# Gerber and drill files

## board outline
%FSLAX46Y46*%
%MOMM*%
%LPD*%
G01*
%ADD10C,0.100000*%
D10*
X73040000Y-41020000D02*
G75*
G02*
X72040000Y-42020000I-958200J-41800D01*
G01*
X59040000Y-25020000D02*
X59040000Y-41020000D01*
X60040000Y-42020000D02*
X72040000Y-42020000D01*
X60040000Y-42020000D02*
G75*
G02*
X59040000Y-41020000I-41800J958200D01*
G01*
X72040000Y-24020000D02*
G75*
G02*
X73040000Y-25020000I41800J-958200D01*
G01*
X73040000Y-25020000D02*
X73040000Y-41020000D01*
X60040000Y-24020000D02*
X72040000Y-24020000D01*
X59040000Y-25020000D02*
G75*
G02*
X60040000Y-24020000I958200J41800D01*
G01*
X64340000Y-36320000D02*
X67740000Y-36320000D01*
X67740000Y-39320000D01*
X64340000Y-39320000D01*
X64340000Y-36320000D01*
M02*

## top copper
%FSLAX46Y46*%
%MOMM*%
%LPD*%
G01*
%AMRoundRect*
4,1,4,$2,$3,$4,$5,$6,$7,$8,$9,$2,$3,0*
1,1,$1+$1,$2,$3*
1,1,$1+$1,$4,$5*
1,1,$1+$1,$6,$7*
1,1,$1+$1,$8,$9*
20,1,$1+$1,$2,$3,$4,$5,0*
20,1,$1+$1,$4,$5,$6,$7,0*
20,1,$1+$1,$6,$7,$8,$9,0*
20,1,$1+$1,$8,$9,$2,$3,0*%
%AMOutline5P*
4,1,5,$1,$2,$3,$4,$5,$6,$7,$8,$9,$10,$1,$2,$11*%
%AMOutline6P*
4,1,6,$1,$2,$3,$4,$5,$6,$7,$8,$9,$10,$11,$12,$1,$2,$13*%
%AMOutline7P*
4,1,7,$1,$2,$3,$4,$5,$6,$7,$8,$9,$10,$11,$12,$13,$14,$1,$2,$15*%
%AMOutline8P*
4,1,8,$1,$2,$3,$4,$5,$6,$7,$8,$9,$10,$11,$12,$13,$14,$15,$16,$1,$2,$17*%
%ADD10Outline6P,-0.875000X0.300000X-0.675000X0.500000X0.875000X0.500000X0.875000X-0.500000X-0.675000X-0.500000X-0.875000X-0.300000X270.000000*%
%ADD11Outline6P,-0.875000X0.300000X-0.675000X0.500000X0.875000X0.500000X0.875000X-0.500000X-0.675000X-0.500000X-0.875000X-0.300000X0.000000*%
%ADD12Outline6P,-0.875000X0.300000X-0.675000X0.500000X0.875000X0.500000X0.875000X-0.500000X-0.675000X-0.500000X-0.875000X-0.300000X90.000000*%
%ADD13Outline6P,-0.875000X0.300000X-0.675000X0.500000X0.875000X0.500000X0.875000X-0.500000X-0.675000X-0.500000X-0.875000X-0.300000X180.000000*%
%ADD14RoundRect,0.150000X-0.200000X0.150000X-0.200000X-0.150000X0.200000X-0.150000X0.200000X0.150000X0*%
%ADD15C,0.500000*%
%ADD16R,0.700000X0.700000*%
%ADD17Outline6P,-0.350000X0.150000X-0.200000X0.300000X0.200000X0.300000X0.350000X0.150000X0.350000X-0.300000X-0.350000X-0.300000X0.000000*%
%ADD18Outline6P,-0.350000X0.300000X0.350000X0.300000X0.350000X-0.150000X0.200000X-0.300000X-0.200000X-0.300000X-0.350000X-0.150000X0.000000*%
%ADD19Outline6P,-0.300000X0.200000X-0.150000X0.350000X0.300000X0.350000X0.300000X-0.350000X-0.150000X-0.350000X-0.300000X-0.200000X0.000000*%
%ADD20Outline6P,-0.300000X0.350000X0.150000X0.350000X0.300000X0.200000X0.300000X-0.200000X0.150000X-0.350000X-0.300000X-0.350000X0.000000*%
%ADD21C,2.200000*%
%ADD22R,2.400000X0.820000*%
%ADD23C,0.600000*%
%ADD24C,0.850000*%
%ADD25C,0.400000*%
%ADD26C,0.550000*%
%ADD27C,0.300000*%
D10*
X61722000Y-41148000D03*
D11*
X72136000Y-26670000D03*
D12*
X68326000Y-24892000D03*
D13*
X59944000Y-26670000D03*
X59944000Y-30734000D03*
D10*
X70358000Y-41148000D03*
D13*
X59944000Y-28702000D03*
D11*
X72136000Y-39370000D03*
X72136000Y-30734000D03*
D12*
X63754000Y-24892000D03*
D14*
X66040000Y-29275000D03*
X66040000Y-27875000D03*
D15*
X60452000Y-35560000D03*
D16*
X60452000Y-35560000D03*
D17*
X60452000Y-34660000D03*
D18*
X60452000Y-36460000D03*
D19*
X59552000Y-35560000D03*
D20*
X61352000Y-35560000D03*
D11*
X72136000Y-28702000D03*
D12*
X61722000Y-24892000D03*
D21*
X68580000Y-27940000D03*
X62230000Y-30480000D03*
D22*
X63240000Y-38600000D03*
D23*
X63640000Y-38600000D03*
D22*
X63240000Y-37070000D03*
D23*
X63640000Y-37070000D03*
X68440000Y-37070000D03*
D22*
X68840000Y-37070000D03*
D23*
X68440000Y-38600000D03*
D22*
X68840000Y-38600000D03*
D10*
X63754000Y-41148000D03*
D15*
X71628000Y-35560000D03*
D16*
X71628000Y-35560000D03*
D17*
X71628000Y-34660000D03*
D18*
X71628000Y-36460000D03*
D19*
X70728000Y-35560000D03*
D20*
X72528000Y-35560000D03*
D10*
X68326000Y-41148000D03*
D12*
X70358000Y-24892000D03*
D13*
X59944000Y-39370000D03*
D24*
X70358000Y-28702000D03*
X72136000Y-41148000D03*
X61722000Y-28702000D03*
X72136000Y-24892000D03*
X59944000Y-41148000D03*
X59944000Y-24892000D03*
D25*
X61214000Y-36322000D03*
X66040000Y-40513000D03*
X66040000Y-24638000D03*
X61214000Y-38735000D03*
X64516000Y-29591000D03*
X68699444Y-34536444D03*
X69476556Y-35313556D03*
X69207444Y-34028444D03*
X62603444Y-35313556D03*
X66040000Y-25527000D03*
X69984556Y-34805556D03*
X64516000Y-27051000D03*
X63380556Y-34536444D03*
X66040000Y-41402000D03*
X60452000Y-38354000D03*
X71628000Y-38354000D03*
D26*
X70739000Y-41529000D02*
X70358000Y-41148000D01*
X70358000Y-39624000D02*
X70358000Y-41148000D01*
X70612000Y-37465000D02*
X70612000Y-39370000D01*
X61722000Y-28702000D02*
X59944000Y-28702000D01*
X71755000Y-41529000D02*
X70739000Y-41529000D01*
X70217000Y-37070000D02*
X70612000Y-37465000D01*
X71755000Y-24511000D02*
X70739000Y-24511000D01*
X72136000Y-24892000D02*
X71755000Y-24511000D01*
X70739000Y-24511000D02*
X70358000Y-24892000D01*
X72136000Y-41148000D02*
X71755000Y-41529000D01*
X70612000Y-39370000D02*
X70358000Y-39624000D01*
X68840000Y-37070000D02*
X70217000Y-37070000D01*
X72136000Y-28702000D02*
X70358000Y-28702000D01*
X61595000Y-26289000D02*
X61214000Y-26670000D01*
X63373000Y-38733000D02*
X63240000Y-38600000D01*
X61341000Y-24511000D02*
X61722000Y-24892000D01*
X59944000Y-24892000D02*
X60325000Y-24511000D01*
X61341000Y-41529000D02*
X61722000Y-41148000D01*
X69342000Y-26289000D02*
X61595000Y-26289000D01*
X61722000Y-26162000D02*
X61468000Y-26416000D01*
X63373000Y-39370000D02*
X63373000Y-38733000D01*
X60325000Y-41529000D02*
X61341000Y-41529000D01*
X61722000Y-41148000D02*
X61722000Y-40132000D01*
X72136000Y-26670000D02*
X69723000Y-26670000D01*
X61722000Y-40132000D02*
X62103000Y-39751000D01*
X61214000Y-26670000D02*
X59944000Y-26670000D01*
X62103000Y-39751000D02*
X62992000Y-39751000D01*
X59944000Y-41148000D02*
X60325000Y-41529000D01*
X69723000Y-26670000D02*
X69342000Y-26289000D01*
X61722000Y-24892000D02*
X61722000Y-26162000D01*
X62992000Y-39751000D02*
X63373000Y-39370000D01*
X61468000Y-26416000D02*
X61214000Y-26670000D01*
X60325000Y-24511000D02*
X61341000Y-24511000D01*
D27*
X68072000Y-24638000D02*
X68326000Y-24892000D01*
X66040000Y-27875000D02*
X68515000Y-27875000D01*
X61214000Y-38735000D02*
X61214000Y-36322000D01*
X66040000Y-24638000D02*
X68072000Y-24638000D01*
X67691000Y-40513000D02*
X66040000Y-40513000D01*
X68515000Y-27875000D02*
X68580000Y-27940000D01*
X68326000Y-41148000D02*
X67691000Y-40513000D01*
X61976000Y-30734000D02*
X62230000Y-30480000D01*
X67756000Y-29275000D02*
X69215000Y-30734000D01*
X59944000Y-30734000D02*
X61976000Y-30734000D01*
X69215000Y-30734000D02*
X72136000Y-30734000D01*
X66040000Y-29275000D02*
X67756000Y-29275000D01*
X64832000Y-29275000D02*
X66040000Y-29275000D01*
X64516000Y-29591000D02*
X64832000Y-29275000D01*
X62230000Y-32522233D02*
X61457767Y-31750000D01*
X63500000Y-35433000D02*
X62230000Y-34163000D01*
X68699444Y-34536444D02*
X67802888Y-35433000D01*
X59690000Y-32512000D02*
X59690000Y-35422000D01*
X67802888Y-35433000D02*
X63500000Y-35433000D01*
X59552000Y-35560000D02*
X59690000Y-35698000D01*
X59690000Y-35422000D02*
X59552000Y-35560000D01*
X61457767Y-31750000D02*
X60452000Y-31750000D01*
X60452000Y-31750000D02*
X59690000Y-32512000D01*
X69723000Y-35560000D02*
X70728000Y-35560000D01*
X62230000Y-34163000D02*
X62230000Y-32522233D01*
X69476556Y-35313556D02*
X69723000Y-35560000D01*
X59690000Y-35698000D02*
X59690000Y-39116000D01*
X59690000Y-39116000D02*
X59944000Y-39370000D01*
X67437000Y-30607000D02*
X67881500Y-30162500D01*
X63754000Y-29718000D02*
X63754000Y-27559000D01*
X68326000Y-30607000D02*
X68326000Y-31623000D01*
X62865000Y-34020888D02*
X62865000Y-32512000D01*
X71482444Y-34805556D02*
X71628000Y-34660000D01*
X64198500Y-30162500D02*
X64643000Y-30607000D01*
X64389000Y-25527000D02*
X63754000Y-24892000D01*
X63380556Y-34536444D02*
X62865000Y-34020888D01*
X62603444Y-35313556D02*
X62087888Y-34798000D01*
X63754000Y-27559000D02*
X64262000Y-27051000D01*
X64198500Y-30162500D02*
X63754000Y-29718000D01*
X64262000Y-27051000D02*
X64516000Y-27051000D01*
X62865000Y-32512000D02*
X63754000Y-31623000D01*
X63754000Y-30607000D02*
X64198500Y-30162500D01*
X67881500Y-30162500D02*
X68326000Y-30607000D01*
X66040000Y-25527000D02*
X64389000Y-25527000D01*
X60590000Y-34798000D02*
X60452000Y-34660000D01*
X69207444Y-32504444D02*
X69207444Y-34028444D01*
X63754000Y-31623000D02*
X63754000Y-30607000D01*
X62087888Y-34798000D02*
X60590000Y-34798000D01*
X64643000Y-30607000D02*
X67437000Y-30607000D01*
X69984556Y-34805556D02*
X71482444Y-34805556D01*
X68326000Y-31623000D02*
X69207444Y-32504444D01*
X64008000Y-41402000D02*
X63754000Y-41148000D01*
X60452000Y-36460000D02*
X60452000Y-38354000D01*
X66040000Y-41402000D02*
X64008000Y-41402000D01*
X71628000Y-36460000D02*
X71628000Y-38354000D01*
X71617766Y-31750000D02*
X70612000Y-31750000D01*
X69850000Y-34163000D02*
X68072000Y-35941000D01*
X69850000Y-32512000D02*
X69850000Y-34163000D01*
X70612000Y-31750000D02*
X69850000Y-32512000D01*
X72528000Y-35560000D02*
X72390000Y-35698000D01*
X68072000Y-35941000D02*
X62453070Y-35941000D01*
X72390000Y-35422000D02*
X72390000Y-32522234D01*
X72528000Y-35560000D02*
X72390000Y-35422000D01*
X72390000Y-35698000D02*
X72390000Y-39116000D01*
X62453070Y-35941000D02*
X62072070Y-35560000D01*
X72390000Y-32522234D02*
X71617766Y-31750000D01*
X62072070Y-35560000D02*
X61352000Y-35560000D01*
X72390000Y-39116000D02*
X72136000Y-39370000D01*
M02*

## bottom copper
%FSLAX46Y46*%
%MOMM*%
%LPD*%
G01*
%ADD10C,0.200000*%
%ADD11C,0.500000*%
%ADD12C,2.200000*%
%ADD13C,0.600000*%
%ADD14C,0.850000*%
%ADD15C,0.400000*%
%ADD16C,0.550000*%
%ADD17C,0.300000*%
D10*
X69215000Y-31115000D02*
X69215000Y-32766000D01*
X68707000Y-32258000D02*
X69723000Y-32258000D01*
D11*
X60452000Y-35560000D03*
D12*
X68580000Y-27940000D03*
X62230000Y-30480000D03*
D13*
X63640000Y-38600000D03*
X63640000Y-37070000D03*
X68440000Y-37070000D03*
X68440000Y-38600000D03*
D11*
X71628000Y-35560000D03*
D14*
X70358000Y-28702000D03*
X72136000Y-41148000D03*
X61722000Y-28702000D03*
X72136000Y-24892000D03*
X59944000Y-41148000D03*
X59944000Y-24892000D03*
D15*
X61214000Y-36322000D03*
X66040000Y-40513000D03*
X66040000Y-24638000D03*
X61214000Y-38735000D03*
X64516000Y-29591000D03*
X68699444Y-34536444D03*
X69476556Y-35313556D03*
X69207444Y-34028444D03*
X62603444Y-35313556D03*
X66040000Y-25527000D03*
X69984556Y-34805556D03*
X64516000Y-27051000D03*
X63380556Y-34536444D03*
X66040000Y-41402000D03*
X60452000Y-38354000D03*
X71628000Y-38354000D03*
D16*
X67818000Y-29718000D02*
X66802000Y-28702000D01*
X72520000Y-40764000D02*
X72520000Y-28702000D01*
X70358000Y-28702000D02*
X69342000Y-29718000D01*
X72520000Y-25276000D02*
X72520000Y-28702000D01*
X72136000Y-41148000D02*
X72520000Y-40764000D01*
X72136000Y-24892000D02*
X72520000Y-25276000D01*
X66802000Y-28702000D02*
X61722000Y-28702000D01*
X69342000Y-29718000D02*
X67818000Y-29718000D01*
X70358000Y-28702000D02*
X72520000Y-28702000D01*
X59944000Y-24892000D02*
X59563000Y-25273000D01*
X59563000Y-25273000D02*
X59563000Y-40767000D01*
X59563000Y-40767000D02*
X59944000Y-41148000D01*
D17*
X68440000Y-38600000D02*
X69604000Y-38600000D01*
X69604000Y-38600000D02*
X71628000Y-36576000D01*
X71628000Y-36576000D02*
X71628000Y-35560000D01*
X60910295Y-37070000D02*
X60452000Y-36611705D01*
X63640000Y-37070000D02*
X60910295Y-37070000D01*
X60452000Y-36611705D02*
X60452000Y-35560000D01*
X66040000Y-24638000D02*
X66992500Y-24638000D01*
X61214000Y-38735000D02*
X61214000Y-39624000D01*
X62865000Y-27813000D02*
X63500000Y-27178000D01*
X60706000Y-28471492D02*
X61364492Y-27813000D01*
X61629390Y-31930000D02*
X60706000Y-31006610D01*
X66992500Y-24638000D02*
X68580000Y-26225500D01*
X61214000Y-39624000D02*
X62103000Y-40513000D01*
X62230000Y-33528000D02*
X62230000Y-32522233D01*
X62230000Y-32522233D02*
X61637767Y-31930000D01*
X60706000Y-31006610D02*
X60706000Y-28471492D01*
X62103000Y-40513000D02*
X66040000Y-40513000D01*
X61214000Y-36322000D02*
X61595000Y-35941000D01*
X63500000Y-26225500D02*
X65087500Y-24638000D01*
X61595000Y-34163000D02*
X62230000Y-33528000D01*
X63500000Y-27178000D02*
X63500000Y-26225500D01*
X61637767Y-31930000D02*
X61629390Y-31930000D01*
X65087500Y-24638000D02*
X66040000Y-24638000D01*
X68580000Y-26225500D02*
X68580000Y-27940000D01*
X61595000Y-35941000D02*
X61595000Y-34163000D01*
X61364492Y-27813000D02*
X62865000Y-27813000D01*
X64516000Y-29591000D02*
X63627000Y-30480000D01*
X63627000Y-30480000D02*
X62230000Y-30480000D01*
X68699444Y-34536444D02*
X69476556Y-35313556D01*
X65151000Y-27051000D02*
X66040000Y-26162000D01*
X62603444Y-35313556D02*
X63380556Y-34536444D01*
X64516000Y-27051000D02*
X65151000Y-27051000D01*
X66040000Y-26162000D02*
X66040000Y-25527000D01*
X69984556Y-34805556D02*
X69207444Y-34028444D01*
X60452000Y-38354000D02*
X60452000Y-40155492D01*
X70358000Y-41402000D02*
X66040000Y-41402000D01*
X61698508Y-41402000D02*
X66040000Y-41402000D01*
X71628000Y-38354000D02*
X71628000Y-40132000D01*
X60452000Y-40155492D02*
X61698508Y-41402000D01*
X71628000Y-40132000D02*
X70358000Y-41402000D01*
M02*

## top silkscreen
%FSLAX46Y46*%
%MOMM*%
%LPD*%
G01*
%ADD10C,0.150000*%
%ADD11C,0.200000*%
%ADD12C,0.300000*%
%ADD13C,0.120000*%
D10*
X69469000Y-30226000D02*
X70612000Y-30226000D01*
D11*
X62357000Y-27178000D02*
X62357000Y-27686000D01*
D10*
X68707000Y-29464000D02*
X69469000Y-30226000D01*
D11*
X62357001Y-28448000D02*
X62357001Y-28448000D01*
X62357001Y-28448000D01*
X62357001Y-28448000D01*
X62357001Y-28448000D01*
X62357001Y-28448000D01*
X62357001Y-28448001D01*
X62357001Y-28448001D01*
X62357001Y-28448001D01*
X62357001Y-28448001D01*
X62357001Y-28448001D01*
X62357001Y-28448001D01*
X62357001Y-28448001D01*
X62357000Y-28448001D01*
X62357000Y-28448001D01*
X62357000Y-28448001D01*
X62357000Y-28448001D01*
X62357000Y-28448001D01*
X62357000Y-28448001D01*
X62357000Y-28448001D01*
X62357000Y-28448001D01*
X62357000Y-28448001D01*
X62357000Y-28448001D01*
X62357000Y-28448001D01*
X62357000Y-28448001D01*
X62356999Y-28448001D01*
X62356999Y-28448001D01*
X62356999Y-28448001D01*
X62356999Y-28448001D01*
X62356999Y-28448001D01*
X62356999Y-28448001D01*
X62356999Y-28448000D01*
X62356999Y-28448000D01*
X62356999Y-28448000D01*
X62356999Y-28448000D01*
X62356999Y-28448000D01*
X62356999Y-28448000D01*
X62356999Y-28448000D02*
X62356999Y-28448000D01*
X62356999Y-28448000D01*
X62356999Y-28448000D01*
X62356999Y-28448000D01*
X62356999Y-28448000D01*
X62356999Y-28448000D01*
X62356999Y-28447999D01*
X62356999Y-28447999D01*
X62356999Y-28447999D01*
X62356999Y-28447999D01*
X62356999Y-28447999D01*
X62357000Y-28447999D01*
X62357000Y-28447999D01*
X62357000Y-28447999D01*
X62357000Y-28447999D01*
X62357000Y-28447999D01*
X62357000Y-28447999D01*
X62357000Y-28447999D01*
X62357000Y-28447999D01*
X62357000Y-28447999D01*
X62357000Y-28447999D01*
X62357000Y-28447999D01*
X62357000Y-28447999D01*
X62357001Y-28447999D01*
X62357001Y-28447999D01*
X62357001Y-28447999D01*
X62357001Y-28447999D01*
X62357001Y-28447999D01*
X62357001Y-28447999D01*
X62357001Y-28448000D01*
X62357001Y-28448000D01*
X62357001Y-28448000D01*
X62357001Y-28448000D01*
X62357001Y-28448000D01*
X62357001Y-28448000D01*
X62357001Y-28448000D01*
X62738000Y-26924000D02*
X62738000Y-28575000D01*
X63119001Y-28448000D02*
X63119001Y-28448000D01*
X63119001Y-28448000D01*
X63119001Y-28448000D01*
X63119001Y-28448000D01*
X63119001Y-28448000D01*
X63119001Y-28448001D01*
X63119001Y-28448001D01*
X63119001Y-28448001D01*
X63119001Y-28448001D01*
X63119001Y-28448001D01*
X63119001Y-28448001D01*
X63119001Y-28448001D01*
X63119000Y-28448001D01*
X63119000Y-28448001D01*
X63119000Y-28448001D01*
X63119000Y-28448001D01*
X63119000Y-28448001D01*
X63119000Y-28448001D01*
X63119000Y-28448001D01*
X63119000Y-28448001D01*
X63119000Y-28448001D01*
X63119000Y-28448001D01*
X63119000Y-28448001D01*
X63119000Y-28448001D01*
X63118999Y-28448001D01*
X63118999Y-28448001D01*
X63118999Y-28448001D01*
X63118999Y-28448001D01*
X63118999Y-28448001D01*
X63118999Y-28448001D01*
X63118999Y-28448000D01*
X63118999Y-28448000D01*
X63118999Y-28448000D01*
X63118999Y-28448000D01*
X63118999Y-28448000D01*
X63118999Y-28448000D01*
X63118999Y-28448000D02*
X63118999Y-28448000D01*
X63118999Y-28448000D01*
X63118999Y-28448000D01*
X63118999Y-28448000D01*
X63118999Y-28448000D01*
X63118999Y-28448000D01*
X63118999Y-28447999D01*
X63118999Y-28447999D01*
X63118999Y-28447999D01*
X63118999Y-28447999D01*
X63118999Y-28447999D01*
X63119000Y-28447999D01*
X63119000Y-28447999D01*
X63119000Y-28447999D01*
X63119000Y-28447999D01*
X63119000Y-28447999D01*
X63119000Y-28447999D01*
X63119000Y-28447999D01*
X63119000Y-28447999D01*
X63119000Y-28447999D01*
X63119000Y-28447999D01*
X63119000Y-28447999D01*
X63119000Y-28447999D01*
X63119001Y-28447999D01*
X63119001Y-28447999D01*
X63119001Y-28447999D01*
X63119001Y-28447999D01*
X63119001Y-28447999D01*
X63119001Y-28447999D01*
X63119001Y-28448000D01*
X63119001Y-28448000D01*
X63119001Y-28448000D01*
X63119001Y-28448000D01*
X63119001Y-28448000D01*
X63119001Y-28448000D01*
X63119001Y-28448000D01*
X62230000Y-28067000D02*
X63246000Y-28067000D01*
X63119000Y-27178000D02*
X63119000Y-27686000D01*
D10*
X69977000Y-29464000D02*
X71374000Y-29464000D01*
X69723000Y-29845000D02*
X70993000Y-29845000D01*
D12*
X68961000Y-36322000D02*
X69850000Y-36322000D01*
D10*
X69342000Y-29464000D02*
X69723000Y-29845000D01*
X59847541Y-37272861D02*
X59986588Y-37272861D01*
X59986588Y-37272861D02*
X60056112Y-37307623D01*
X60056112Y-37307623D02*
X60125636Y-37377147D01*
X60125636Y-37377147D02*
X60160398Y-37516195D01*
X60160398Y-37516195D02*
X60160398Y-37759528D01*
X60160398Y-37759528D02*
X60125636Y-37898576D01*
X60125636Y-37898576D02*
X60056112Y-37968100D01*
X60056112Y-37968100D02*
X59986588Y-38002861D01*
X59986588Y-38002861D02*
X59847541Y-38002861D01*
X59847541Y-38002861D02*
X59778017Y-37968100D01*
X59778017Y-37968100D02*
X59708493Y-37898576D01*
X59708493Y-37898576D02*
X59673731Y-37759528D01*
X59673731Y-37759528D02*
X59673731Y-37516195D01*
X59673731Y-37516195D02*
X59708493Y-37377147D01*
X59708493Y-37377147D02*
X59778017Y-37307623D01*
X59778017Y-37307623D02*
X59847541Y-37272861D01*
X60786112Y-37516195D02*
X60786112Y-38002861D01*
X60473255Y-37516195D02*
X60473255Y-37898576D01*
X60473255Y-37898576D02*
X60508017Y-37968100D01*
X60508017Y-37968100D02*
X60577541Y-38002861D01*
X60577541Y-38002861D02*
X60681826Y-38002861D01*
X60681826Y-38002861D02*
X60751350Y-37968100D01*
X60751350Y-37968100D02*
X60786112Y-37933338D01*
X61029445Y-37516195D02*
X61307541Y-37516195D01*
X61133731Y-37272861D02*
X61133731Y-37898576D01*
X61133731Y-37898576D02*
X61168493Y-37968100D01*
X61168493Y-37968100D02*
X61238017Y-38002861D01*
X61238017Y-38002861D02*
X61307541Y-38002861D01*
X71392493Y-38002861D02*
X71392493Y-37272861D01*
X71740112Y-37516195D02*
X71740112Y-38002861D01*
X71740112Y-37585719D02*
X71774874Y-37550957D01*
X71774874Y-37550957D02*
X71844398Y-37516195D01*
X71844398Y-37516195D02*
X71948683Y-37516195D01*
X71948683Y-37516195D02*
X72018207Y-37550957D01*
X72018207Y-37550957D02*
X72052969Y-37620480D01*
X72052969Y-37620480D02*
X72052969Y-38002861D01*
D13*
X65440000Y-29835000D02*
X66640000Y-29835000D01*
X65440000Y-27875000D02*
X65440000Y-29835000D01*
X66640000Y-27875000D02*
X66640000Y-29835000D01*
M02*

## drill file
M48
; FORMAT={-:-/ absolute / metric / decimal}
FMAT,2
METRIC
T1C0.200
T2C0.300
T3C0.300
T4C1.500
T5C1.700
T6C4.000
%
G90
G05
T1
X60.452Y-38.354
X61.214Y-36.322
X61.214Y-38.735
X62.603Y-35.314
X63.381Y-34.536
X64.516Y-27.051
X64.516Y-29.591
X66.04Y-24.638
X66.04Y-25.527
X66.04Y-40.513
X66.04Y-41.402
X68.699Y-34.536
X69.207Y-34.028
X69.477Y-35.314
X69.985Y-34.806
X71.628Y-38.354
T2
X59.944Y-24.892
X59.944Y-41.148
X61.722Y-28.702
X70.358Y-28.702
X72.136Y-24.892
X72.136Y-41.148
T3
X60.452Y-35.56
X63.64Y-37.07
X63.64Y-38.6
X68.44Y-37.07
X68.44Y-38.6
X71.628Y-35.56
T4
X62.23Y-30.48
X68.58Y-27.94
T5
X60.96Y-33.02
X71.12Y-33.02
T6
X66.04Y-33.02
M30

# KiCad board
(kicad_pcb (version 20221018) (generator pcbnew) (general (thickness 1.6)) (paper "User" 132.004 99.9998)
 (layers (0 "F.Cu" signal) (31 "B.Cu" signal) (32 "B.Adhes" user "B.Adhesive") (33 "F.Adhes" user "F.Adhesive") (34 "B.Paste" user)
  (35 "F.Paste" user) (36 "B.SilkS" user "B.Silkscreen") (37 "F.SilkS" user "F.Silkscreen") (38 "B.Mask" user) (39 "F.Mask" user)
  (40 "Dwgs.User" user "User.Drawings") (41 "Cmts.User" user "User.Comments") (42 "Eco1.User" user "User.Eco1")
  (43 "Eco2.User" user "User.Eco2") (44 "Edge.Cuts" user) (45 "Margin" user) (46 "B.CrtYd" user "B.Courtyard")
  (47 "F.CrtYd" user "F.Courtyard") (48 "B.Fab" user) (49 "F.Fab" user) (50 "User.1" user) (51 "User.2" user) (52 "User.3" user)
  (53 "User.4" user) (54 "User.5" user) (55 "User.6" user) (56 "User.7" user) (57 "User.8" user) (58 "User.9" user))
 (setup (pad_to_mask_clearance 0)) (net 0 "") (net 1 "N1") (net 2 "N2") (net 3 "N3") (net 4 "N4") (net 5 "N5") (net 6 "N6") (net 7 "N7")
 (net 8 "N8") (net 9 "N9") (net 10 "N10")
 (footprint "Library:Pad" (layer "F.Cu") (at 61.722 41.148 -90)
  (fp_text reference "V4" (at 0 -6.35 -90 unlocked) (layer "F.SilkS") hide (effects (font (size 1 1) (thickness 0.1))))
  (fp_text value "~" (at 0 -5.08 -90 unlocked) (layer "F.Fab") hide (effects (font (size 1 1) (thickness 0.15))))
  (pad "1" smd roundrect (at 0 0 270) (size 1.75 1) (layers "F.Cu" "F.Paste" "F.Mask") (roundrect_rratio 0) (chamfer_ratio 0.2)
   (chamfer top_left bottom_left) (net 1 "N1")))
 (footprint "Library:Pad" (layer "F.Cu") (at 72.136 26.67)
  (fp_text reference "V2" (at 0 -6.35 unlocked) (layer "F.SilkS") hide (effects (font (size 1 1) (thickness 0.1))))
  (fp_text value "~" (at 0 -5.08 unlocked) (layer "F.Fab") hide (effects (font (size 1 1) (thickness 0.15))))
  (pad "1" smd roundrect (at 0 0) (size 1.75 1) (layers "F.Cu" "F.Paste" "F.Mask") (roundrect_rratio 0) (chamfer_ratio 0.2)
   (chamfer top_left bottom_left) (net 1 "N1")))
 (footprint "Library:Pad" (layer "F.Cu") (at 68.326 24.892 90)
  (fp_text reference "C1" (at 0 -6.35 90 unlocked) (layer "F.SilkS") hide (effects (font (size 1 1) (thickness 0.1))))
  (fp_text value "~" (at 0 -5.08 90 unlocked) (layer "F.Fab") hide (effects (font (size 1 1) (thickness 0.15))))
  (pad "1" smd roundrect (at 0 0 90) (size 1.75 1) (layers "F.Cu" "F.Paste" "F.Mask") (roundrect_rratio 0) (chamfer_ratio 0.2)
   (chamfer top_left bottom_left) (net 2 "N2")))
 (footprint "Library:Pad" (layer "F.Cu") (at 59.944 26.67 180)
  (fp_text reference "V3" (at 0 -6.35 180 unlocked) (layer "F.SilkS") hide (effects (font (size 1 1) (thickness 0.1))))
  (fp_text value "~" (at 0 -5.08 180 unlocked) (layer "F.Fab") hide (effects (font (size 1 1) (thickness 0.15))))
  (pad "1" smd roundrect (at 0 0 180) (size 1.75 1) (layers "F.Cu" "F.Paste" "F.Mask") (roundrect_rratio 0) (chamfer_ratio 0.2)
   (chamfer top_left bottom_left) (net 1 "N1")))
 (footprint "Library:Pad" (layer "F.Cu") (at 59.944 30.734 180)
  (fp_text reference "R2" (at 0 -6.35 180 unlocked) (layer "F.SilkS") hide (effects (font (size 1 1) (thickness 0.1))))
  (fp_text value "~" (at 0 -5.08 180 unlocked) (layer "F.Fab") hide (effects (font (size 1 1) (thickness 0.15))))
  (pad "1" smd roundrect (at 0 0 180) (size 1.75 1) (layers "F.Cu" "F.Paste" "F.Mask") (roundrect_rratio 0) (chamfer_ratio 0.2)
   (chamfer top_left bottom_left) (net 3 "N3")))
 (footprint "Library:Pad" (layer "F.Cu") (at 70.358 41.148 -90)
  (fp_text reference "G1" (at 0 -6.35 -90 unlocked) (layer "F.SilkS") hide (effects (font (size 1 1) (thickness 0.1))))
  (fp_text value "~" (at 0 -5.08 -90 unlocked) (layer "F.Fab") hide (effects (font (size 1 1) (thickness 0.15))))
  (pad "1" smd roundrect (at 0 0 270) (size 1.75 1) (layers "F.Cu" "F.Paste" "F.Mask") (roundrect_rratio 0) (chamfer_ratio 0.2)
   (chamfer top_left bottom_left) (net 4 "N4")))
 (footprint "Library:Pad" (layer "F.Cu") (at 59.944 28.702 180)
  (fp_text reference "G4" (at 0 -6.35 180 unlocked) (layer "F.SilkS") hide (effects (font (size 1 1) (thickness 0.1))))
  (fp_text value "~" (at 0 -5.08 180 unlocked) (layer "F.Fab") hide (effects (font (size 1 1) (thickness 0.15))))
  (pad "1" smd roundrect (at 0 0 180) (size 1.75 1) (layers "F.Cu" "F.Paste" "F.Mask") (roundrect_rratio 0) (chamfer_ratio 0.2)
   (chamfer top_left bottom_left) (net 4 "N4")))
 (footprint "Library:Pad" (layer "F.Cu") (at 72.136 39.37)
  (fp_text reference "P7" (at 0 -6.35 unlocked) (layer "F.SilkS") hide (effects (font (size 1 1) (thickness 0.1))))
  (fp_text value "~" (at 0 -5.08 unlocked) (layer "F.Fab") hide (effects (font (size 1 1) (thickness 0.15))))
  (pad "1" smd roundrect (at 0 0) (size 1.75 1) (layers "F.Cu" "F.Paste" "F.Mask") (roundrect_rratio 0) (chamfer_ratio 0.2)
   (chamfer top_left bottom_left) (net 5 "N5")))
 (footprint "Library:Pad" (layer "F.Cu") (at 72.136 30.734)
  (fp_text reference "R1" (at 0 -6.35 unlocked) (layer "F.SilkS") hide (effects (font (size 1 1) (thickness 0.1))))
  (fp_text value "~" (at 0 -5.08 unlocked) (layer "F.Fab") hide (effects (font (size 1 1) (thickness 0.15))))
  (pad "1" smd roundrect (at 0 0) (size 1.75 1) (layers "F.Cu" "F.Paste" "F.Mask") (roundrect_rratio 0) (chamfer_ratio 0.2)
   (chamfer top_left bottom_left) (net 3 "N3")))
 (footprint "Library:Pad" (layer "F.Cu") (at 63.754 24.892 90)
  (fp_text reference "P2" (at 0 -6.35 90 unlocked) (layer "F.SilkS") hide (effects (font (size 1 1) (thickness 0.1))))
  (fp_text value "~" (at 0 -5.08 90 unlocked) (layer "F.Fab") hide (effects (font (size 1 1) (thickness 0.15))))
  (pad "1" smd roundrect (at 0 0 90) (size 1.75 1) (layers "F.Cu" "F.Paste" "F.Mask") (roundrect_rratio 0) (chamfer_ratio 0.2)
   (chamfer top_left bottom_left) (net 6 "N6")))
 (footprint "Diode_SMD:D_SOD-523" (layer "F.Cu") (at 66.04 28.575 90)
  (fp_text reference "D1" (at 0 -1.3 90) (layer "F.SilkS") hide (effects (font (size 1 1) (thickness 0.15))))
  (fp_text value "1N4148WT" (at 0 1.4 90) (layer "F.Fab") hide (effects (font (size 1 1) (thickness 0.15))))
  (fp_line (start -1.26 -0.6) (end -1.26 0.6) (stroke (width 0.12) (type solid)) (layer "F.SilkS"))
  (fp_line (start 0.7 -0.6) (end -1.26 -0.6) (stroke (width 0.12) (type solid)) (layer "F.SilkS"))
  (fp_line (start 0.7 0.6) (end -1.26 0.6) (stroke (width 0.12) (type solid)) (layer "F.SilkS"))
  (pad "1" smd roundrect (at -0.7 0 270) (size 0.6 0.7) (layers "F.Cu" "F.Paste" "F.Mask") (roundrect_rratio 0.25) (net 3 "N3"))
  (pad "2" smd roundrect (at 0.7 0 270) (size 0.6 0.7) (layers "F.Cu" "F.Paste" "F.Mask") (roundrect_rratio 0.25) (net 2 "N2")))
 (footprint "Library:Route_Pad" (layer "F.Cu") (at 60.452 35.56)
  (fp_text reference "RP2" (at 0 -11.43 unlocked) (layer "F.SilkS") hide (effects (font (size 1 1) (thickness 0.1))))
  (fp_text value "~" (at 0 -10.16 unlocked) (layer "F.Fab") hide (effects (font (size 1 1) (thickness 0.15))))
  (pad "1" thru_hole circle (at 0 0) (size 0.5 0.5) (drill 0.3) (layers "*.Cu" "*.Mask") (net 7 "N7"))
  (pad "1" smd rect (at 0 0) (size 0.7 0.7) (layers "F.Cu" "F.Paste" "F.Mask") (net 7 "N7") (thermal_bridge_angle 45))
  (pad "2" smd roundrect (at 0 -0.9) (size 0.7 0.6) (layers "F.Cu" "F.Paste" "F.Mask") (roundrect_rratio 0) (chamfer_ratio 0.25)
   (chamfer top_left top_right) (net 6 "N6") (thermal_bridge_angle 45))
  (pad "3" smd roundrect (at 0 0.9) (size 0.7 0.6) (layers "F.Cu" "F.Paste" "F.Mask") (roundrect_rratio 0) (chamfer_ratio 0.25)
   (chamfer bottom_left bottom_right) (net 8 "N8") (thermal_bridge_angle 45))
  (pad "4" smd roundrect (at -0.9 0) (size 0.6 0.7) (layers "F.Cu" "F.Paste" "F.Mask") (roundrect_rratio 0) (chamfer_ratio 0.25)
   (chamfer top_left bottom_left) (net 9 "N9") (thermal_bridge_angle 45))
  (pad "5" smd roundrect (at 0.9 0) (size 0.6 0.7) (layers "F.Cu" "F.Paste" "F.Mask") (roundrect_rratio 0) (chamfer_ratio 0.25)
   (chamfer top_right bottom_right) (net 5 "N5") (thermal_bridge_angle 45)))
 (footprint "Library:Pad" (layer "F.Cu") (at 72.136 28.702)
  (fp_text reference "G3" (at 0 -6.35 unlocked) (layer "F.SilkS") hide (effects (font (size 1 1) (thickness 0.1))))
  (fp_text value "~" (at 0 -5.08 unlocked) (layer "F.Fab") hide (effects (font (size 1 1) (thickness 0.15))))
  (pad "1" smd roundrect (at 0 0) (size 1.75 1) (layers "F.Cu" "F.Paste" "F.Mask") (roundrect_rratio 0) (chamfer_ratio 0.2)
   (chamfer top_left bottom_left) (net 4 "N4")))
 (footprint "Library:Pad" (layer "F.Cu") (at 61.722 24.892 90)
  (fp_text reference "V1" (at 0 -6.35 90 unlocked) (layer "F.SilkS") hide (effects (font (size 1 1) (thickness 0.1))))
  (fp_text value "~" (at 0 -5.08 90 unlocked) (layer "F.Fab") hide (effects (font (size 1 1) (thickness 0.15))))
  (pad "1" smd roundrect (at 0 0 90) (size 1.75 1) (layers "F.Cu" "F.Paste" "F.Mask") (roundrect_rratio 0) (chamfer_ratio 0.2)
   (chamfer top_left bottom_left) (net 1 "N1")))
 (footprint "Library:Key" (layer "F.Cu") (at 66.04 33.02)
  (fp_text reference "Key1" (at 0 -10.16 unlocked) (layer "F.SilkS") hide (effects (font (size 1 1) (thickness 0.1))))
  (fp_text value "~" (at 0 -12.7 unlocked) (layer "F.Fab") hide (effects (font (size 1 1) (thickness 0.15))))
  (fp_rect (start -1.7 3.3) (end 1.7 6.3) (stroke (width 0.1) (type default)) (fill none) (layer "Edge.Cuts"))
  (pad "" np_thru_hole circle (at -5.08 0) (size 1.7 1.7) (drill 1.7) (layers "F&B.Cu" "*.Mask"))
  (pad "" np_thru_hole circle (at 0 0) (size 4 4) (drill 4) (layers "F&B.Cu" "*.Mask"))
  (pad "" np_thru_hole circle (at 5.08 0) (size 1.7 1.7) (drill 1.7) (layers "F&B.Cu" "*.Mask"))
  (pad "1" thru_hole circle (at 2.54 -5.08) (size 2.2 2.2) (drill 1.5) (layers "*.Cu" "*.Mask") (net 2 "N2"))
  (pad "2" thru_hole circle (at -3.81 -2.54) (size 2.2 2.2) (drill 1.5) (layers "*.Cu" "*.Mask") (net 3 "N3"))
  (pad "3" smd rect (at -2.8 5.58) (size 2.4 0.82) (layers "F.Cu" "F.Paste" "F.Mask") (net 1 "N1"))
  (pad "3" thru_hole circle (at -2.4 5.58) (size 0.6 0.6) (drill 0.3) (layers "*.Cu" "*.Mask") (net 1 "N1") (thermal_bridge_angle 90))
  (pad "4" smd rect (at -2.8 4.05) (size 2.4 0.82) (layers "F.Cu" "F.Paste" "F.Mask") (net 7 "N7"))
  (pad "4" thru_hole circle (at -2.4 4.05) (size 0.6 0.6) (drill 0.3) (layers "*.Cu" "*.Mask") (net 7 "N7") (thermal_bridge_angle 90))
  (pad "5" thru_hole circle (at 2.4 4.05) (size 0.6 0.6) (drill 0.3) (layers "*.Cu" "*.Mask") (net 4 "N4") (thermal_bridge_angle 90))
  (pad "5" smd rect (at 2.8 4.05) (size 2.4 0.82) (layers "F.Cu" "F.Paste" "F.Mask") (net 4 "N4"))
  (pad "6" thru_hole circle (at 2.4 5.58) (size 0.6 0.6) (drill 0.3) (layers "*.Cu" "*.Mask") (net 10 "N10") (thermal_bridge_angle 90))
  (pad "6" smd rect (at 2.8 5.58) (size 2.4 0.82) (layers "F.Cu" "F.Paste" "F.Mask") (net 10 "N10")))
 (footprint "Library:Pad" (layer "F.Cu") (at 63.754 41.148 -90)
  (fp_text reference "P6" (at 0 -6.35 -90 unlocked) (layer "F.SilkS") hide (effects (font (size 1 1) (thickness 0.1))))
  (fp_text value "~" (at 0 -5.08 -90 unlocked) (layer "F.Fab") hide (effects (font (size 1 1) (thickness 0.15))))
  (pad "1" smd roundrect (at 0 0 270) (size 1.75 1) (layers "F.Cu" "F.Paste" "F.Mask") (roundrect_rratio 0) (chamfer_ratio 0.2)
   (chamfer top_left bottom_left) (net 8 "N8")))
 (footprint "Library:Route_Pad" (layer "F.Cu") (at 71.628 35.56)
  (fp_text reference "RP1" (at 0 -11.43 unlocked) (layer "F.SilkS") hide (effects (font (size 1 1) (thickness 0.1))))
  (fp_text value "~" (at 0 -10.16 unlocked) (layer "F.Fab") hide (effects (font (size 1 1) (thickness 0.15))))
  (pad "1" thru_hole circle (at 0 0) (size 0.5 0.5) (drill 0.3) (layers "*.Cu" "*.Mask") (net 10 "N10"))
  (pad "1" smd rect (at 0 0) (size 0.7 0.7) (layers "F.Cu" "F.Paste" "F.Mask") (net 10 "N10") (thermal_bridge_angle 45))
  (pad "2" smd roundrect (at 0 -0.9) (size 0.7 0.6) (layers "F.Cu" "F.Paste" "F.Mask") (roundrect_rratio 0) (chamfer_ratio 0.25)
   (chamfer top_left top_right) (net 6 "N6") (thermal_bridge_angle 45))
  (pad "3" smd roundrect (at 0 0.9) (size 0.7 0.6) (layers "F.Cu" "F.Paste" "F.Mask") (roundrect_rratio 0) (chamfer_ratio 0.25)
   (chamfer bottom_left bottom_right) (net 8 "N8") (thermal_bridge_angle 45))
  (pad "4" smd roundrect (at -0.9 0) (size 0.6 0.7) (layers "F.Cu" "F.Paste" "F.Mask") (roundrect_rratio 0) (chamfer_ratio 0.25)
   (chamfer top_left bottom_left) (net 9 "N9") (thermal_bridge_angle 45))
  (pad "5" smd roundrect (at 0.9 0) (size 0.6 0.7) (layers "F.Cu" "F.Paste" "F.Mask") (roundrect_rratio 0) (chamfer_ratio 0.25)
   (chamfer top_right bottom_right) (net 5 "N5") (thermal_bridge_angle 45)))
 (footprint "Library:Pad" (layer "F.Cu") (at 68.326 41.148 -90)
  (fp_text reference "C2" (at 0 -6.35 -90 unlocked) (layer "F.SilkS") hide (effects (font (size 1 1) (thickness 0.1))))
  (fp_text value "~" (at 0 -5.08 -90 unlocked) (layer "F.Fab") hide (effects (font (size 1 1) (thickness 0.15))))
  (pad "1" smd roundrect (at 0 0 270) (size 1.75 1) (layers "F.Cu" "F.Paste" "F.Mask") (roundrect_rratio 0) (chamfer_ratio 0.2)
   (chamfer top_left bottom_left) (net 2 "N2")))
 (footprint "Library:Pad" (layer "F.Cu") (at 70.358 24.892 90)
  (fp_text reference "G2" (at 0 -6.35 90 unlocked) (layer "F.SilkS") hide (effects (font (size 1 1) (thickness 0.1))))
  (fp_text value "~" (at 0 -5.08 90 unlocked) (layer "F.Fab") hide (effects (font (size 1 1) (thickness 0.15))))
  (pad "1" smd roundrect (at 0 0 90) (size 1.75 1) (layers "F.Cu" "F.Paste" "F.Mask") (roundrect_rratio 0) (chamfer_ratio 0.2)
   (chamfer top_left bottom_left) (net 4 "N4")))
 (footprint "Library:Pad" (layer "F.Cu") (at 59.944 39.37 180)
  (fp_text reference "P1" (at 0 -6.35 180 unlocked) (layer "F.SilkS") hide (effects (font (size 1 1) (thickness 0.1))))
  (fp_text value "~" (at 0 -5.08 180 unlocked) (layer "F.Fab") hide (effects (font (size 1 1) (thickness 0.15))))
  (pad "1" smd roundrect (at 0 0 180) (size 1.75 1) (layers "F.Cu" "F.Paste" "F.Mask") (roundrect_rratio 0) (chamfer_ratio 0.2)
   (chamfer top_left bottom_left) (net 9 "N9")))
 (gr_line (start 69.215 31.115) (end 69.215 32.766) (stroke (width 0.2) (type default)) (layer "B.Cu"))
 (gr_line (start 68.707 32.258) (end 69.723 32.258) (stroke (width 0.2) (type default)) (layer "B.Cu"))
 (gr_line (start 69.469 30.226) (end 70.612 30.226) (stroke (width 0.15) (type default)) (layer "F.SilkS"))
 (gr_line (start 62.357 27.178) (end 62.357 27.686) (stroke (width 0.2) (type default)) (layer "F.SilkS"))
 (gr_line (start 68.707 29.464) (end 69.469 30.226) (stroke (width 0.15) (type default)) (layer "F.SilkS"))
 (gr_circle (center 62.357 28.448) (end 62.357001 28.448) (stroke (width 0.2) (type default)) (fill none) (layer "F.SilkS"))
 (gr_line (start 62.738 26.924) (end 62.738 28.575) (stroke (width 0.2) (type default)) (layer "F.SilkS"))
 (gr_circle (center 63.119 28.448) (end 63.119001 28.448) (stroke (width 0.2) (type default)) (fill none) (layer "F.SilkS"))
 (gr_line (start 62.23 28.067) (end 63.246 28.067) (stroke (width 0.2) (type default)) (layer "F.SilkS"))
 (gr_line (start 63.119 27.178) (end 63.119 27.686) (stroke (width 0.2) (type default)) (layer "F.SilkS"))
 (gr_line (start 69.977 29.464) (end 71.374 29.464) (stroke (width 0.15) (type default)) (layer "F.SilkS"))
 (gr_line (start 69.723 29.845) (end 70.993 29.845) (stroke (width 0.15) (type default)) (layer "F.SilkS"))
 (gr_line (start 68.961 36.322) (end 69.85 36.322) (stroke (width 0.3) (type default)) (layer "F.SilkS"))
 (gr_line (start 69.342 29.464) (end 69.723 29.845) (stroke (width 0.15) (type default)) (layer "F.SilkS"))
 (gr_arc (start 73.04 41.02) (mid 72.759994 41.739993) (end 72.04 42.02) (stroke (width 0.1) (type default)) (layer "Edge.Cuts"))
 (gr_line (start 59.04 25.02) (end 59.04 41.02) (stroke (width 0.1) (type default)) (layer "Edge.Cuts"))
 (gr_line (start 60.04 42.02) (end 72.04 42.02) (stroke (width 0.1) (type default)) (layer "Edge.Cuts"))
 (gr_arc (start 60.04 42.02) (mid 59.320007 41.739994) (end 59.04 41.02) (stroke (width 0.1) (type default)) (layer "Edge.Cuts"))
 (gr_arc (start 72.04 24.02) (mid 72.759993 24.300006) (end 73.04 25.02) (stroke (width 0.1) (type default)) (layer "Edge.Cuts"))
 (gr_line (start 73.04 25.02) (end 73.04 41.02) (stroke (width 0.1) (type default)) (layer "Edge.Cuts"))
 (gr_line (start 60.04 24.02) (end 72.04 24.02) (stroke (width 0.1) (type default)) (layer "Edge.Cuts"))
 (gr_arc (start 59.04 25.02) (mid 59.320006 24.300007) (end 60.04 24.02) (stroke (width 0.1) (type default)) (layer "Edge.Cuts"))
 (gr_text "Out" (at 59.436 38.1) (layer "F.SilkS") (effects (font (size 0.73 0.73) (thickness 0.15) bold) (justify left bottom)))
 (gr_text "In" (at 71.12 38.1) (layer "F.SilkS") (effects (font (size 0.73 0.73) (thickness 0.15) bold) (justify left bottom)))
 (segment (start 70.739 41.529) (end 70.358 41.148) (width 0.55) (layer "F.Cu") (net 4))
 (segment (start 70.358 39.624) (end 70.358 41.148) (width 0.55) (layer "F.Cu") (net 4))
 (segment (start 70.612 37.465) (end 70.612 39.37) (width 0.55) (layer "F.Cu") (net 4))
 (segment (start 61.722 28.702) (end 59.944 28.702) (width 0.55) (layer "F.Cu") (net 4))
 (segment (start 71.755 41.529) (end 70.739 41.529) (width 0.55) (layer "F.Cu") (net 4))
 (segment (start 70.217 37.07) (end 70.612 37.465) (width 0.55) (layer "F.Cu") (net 4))
 (segment (start 71.755 24.511) (end 70.739 24.511) (width 0.55) (layer "F.Cu") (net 4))
 (segment (start 72.136 24.892) (end 71.755 24.511) (width 0.55) (layer "F.Cu") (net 4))
 (segment (start 70.739 24.511) (end 70.358 24.892) (width 0.55) (layer "F.Cu") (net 4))
 (segment (start 72.136 41.148) (end 71.755 41.529) (width 0.55) (layer "F.Cu") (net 4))
 (segment (start 70.612 39.37) (end 70.358 39.624) (width 0.55) (layer "F.Cu") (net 4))
 (segment (start 68.84 37.07) (end 70.217 37.07) (width 0.55) (layer "F.Cu") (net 4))
 (segment (start 72.136 28.702) (end 70.358 28.702) (width 0.55) (layer "F.Cu") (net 4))
 (via (at 70.358 28.702) (size 0.85) (drill 0.3) (layers "F.Cu" "B.Cu") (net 4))
 (via (at 72.136 41.148) (size 0.85) (drill 0.3) (layers "F.Cu" "B.Cu") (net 4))
 (via (at 61.722 28.702) (size 0.85) (drill 0.3) (layers "F.Cu" "B.Cu") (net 4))
 (via (at 72.136 24.892) (size 0.85) (drill 0.3) (layers "F.Cu" "B.Cu") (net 4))
 (segment (start 67.818 29.718) (end 66.802 28.702) (width 0.55) (layer "B.Cu") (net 4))
 (segment (start 72.52 40.764) (end 72.52 28.702) (width 0.55) (layer "B.Cu") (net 4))
 (segment (start 70.358 28.702) (end 69.342 29.718) (width 0.55) (layer "B.Cu") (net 4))
 (segment (start 72.52 25.276) (end 72.52 28.702) (width 0.55) (layer "B.Cu") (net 4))
 (segment (start 72.136 41.148) (end 72.52 40.764) (width 0.55) (layer "B.Cu") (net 4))
 (segment (start 72.136 24.892) (end 72.52 25.276) (width 0.55) (layer "B.Cu") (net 4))
 (segment (start 66.802 28.702) (end 61.722 28.702) (width 0.55) (layer "B.Cu") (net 4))
 (segment (start 69.342 29.718) (end 67.818 29.718) (width 0.55) (layer "B.Cu") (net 4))
 (segment (start 70.358 28.702) (end 72.52 28.702) (width 0.55) (layer "B.Cu") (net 4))
 (segment (start 61.595 26.289) (end 61.214 26.67) (width 0.55) (layer "F.Cu") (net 1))
 (segment (start 63.373 38.733) (end 63.24 38.6) (width 0.55) (layer "F.Cu") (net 1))
 (segment (start 61.341 24.511) (end 61.722 24.892) (width 0.55) (layer "F.Cu") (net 1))
 (segment (start 59.944 24.892) (end 60.325 24.511) (width 0.55) (layer "F.Cu") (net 1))
 (segment (start 61.341 41.529) (end 61.722 41.148) (width 0.55) (layer "F.Cu") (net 1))
 (segment (start 69.342 26.289) (end 61.595 26.289) (width 0.55) (layer "F.Cu") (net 1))
 (segment (start 61.722 26.162) (end 61.468 26.416) (width 0.55) (layer "F.Cu") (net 1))
 (segment (start 63.373 39.37) (end 63.373 38.733) (width 0.55) (layer "F.Cu") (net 1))
 (segment (start 60.325 41.529) (end 61.341 41.529) (width 0.55) (layer "F.Cu") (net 1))
 (segment (start 61.722 41.148) (end 61.722 40.132) (width 0.55) (layer "F.Cu") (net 1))
 (segment (start 72.136 26.67) (end 69.723 26.67) (width 0.55) (layer "F.Cu") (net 1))
 (segment (start 61.722 40.132) (end 62.103 39.751) (width 0.55) (layer "F.Cu") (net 1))
 (segment (start 61.214 26.67) (end 59.944 26.67) (width 0.55) (layer "F.Cu") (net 1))
 (segment (start 62.103 39.751) (end 62.992 39.751) (width 0.55) (layer "F.Cu") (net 1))
 (segment (start 59.944 41.148) (end 60.325 41.529) (width 0.55) (layer "F.Cu") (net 1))
 (segment (start 69.723 26.67) (end 69.342 26.289) (width 0.55) (layer "F.Cu") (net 1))
 (segment (start 61.722 24.892) (end 61.722 26.162) (width 0.55) (layer "F.Cu") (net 1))
 (segment (start 62.992 39.751) (end 63.373 39.37) (width 0.55) (layer "F.Cu") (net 1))
 (segment (start 61.468 26.416) (end 61.214 26.67) (width 0.55) (layer "F.Cu") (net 1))
 (segment (start 60.325 24.511) (end 61.341 24.511) (width 0.55) (layer "F.Cu") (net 1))
 (via (at 59.944 41.148) (size 0.85) (drill 0.3) (layers "F.Cu" "B.Cu") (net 1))
 (via (at 59.944 24.892) (size 0.85) (drill 0.3) (layers "F.Cu" "B.Cu") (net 1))
 (segment (start 59.944 24.892) (end 59.563 25.273) (width 0.55) (layer "B.Cu") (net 1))
 (segment (start 59.563 25.273) (end 59.563 40.767) (width 0.55) (layer "B.Cu") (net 1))
 (segment (start 59.563 40.767) (end 59.944 41.148) (width 0.55) (layer "B.Cu") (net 1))
 (segment (start 68.44 38.6) (end 69.604 38.6) (width 0.3) (layer "B.Cu") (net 10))
 (segment (start 69.604 38.6) (end 71.628 36.576) (width 0.3) (layer "B.Cu") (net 10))
 (segment (start 71.628 36.576) (end 71.628 35.56) (width 0.3) (layer "B.Cu") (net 10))
 (segment (start 60.910295 37.07) (end 60.452 36.611705) (width 0.3) (layer "B.Cu") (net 7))
 (segment (start 63.64 37.07) (end 60.910295 37.07) (width 0.3) (layer "B.Cu") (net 7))
 (segment (start 60.452 36.611705) (end 60.452 35.56) (width 0.3) (layer "B.Cu") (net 7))
 (segment (start 68.072 24.638) (end 68.326 24.892) (width 0.3) (layer "F.Cu") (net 2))
 (segment (start 66.04 27.875) (end 68.515 27.875) (width 0.3) (layer "F.Cu") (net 2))
 (segment (start 61.214 38.735) (end 61.214 36.322) (width 0.3) (layer "F.Cu") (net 2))
 (segment (start 66.04 24.638) (end 68.072 24.638) (width 0.3) (layer "F.Cu") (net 2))
 (segment (start 67.691 40.513) (end 66.04 40.513) (width 0.3) (layer "F.Cu") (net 2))
 (segment (start 68.515 27.875) (end 68.58 27.94) (width 0.3) (layer "F.Cu") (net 2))
 (segment (start 68.326 41.148) (end 67.691 40.513) (width 0.3) (layer "F.Cu") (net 2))
 (via (at 61.214 36.322) (size 0.4) (drill 0.2) (layers "F.Cu" "B.Cu") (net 2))
 (via (at 66.04 40.513) (size 0.4) (drill 0.2) (layers "F.Cu" "B.Cu") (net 2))
 (via (at 66.04 24.638) (size 0.4) (drill 0.2) (layers "F.Cu" "B.Cu") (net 2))
 (via (at 61.214 38.735) (size 0.4) (drill 0.2) (layers "F.Cu" "B.Cu") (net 2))
 (segment (start 66.04 24.638) (end 66.9925 24.638) (width 0.3) (layer "B.Cu") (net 2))
 (segment (start 61.214 38.735) (end 61.214 39.624) (width 0.3) (layer "B.Cu") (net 2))
 (segment (start 62.865 27.813) (end 63.5 27.178) (width 0.3) (layer "B.Cu") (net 2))
 (segment (start 60.706 28.471492) (end 61.364492 27.813) (width 0.3) (layer "B.Cu") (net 2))
 (segment (start 61.62939 31.93) (end 60.706 31.00661) (width 0.3) (layer "B.Cu") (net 2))
 (segment (start 66.9925 24.638) (end 68.58 26.2255) (width 0.3) (layer "B.Cu") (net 2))
 (segment (start 61.214 39.624) (end 62.103 40.513) (width 0.3) (layer "B.Cu") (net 2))
 (segment (start 62.23 33.528) (end 62.23 32.522233) (width 0.3) (layer "B.Cu") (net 2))
 (segment (start 62.23 32.522233) (end 61.637767 31.93) (width 0.3) (layer "B.Cu") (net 2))
 (segment (start 60.706 31.00661) (end 60.706 28.471492) (width 0.3) (layer "B.Cu") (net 2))
 (segment (start 62.103 40.513) (end 66.04 40.513) (width 0.3) (layer "B.Cu") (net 2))
 (segment (start 61.214 36.322) (end 61.595 35.941) (width 0.3) (layer "B.Cu") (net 2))
 (segment (start 63.5 26.2255) (end 65.0875 24.638) (width 0.3) (layer "B.Cu") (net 2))
 (segment (start 61.595 34.163) (end 62.23 33.528) (width 0.3) (layer "B.Cu") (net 2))
 (segment (start 63.5 27.178) (end 63.5 26.2255) (width 0.3) (layer "B.Cu") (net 2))
 (segment (start 61.637767 31.93) (end 61.62939 31.93) (width 0.3) (layer "B.Cu") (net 2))
 (segment (start 65.0875 24.638) (end 66.04 24.638) (width 0.3) (layer "B.Cu") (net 2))
 (segment (start 68.58 26.2255) (end 68.58 27.94) (width 0.3) (layer "B.Cu") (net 2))
 (segment (start 61.595 35.941) (end 61.595 34.163) (width 0.3) (layer "B.Cu") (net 2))
 (segment (start 61.364492 27.813) (end 62.865 27.813) (width 0.3) (layer "B.Cu") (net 2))
 (segment (start 61.976 30.734) (end 62.23 30.48) (width 0.3) (layer "F.Cu") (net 3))
 (segment (start 67.756 29.275) (end 69.215 30.734) (width 0.3) (layer "F.Cu") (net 3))
 (segment (start 59.944 30.734) (end 61.976 30.734) (width 0.3) (layer "F.Cu") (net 3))
 (segment (start 69.215 30.734) (end 72.136 30.734) (width 0.3) (layer "F.Cu") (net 3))
 (segment (start 66.04 29.275) (end 67.756 29.275) (width 0.3) (layer "F.Cu") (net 3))
 (segment (start 64.832 29.275) (end 66.04 29.275) (width 0.3) (layer "F.Cu") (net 3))
 (segment (start 64.516 29.591) (end 64.832 29.275) (width 0.3) (layer "F.Cu") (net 3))
 (via (at 64.516 29.591) (size 0.4) (drill 0.2) (layers "F.Cu" "B.Cu") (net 3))
 (segment (start 64.516 29.591) (end 63.627 30.48) (width 0.3) (layer "B.Cu") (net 3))
 (segment (start 63.627 30.48) (end 62.23 30.48) (width 0.3) (layer "B.Cu") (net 3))
 (segment (start 62.23 32.522233) (end 61.457767 31.75) (width 0.3) (layer "F.Cu") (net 9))
 (segment (start 63.5 35.433) (end 62.23 34.163) (width 0.3) (layer "F.Cu") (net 9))
 (segment (start 68.699444 34.536444) (end 67.802888 35.433) (width 0.3) (layer "F.Cu") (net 9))
 (segment (start 59.69 32.512) (end 59.69 35.422) (width 0.3) (layer "F.Cu") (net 9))
 (segment (start 67.802888 35.433) (end 63.5 35.433) (width 0.3) (layer "F.Cu") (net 9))
 (segment (start 59.552 35.56) (end 59.69 35.698) (width 0.3) (layer "F.Cu") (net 9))
 (segment (start 59.69 35.422) (end 59.552 35.56) (width 0.3) (layer "F.Cu") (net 9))
 (segment (start 61.457767 31.75) (end 60.452 31.75) (width 0.3) (layer "F.Cu") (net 9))
 (segment (start 60.452 31.75) (end 59.69 32.512) (width 0.3) (layer "F.Cu") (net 9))
 (segment (start 69.723 35.56) (end 70.728 35.56) (width 0.3) (layer "F.Cu") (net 9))
 (segment (start 62.23 34.163) (end 62.23 32.522233) (width 0.3) (layer "F.Cu") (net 9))
 (segment (start 69.476556 35.313556) (end 69.723 35.56) (width 0.3) (layer "F.Cu") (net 9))
 (segment (start 59.69 35.698) (end 59.69 39.116) (width 0.3) (layer "F.Cu") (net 9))
 (segment (start 59.69 39.116) (end 59.944 39.37) (width 0.3) (layer "F.Cu") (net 9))
 (via (at 68.699444 34.536444) (size 0.4) (drill 0.2) (layers "F.Cu" "B.Cu") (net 9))
 (via (at 69.476556 35.313556) (size 0.4) (drill 0.2) (layers "F.Cu" "B.Cu") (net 9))
 (segment (start 68.699444 34.536444) (end 69.476556 35.313556) (width 0.3) (layer "B.Cu") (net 9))
 (segment (start 67.437 30.607) (end 67.8815 30.1625) (width 0.3) (layer "F.Cu") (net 6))
 (segment (start 63.754 29.718) (end 63.754 27.559) (width 0.3) (layer "F.Cu") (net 6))
 (segment (start 68.326 30.607) (end 68.326 31.623) (width 0.3) (layer "F.Cu") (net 6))
 (segment (start 62.865 34.020888) (end 62.865 32.512) (width 0.3) (layer "F.Cu") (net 6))
 (segment (start 71.482444 34.805556) (end 71.628 34.66) (width 0.3) (layer "F.Cu") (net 6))
 (segment (start 64.1985 30.1625) (end 64.643 30.607) (width 0.3) (layer "F.Cu") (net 6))
 (segment (start 64.389 25.527) (end 63.754 24.892) (width 0.3) (layer "F.Cu") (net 6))
 (segment (start 63.380556 34.536444) (end 62.865 34.020888) (width 0.3) (layer "F.Cu") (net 6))
 (segment (start 62.603444 35.313556) (end 62.087888 34.798) (width 0.3) (layer "F.Cu") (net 6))
 (segment (start 63.754 27.559) (end 64.262 27.051) (width 0.3) (layer "F.Cu") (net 6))
 (segment (start 64.1985 30.1625) (end 63.754 29.718) (width 0.3) (layer "F.Cu") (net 6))
 (segment (start 64.262 27.051) (end 64.516 27.051) (width 0.3) (layer "F.Cu") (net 6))
 (segment (start 62.865 32.512) (end 63.754 31.623) (width 0.3) (layer "F.Cu") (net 6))
 (segment (start 63.754 30.607) (end 64.1985 30.1625) (width 0.3) (layer "F.Cu") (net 6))
 (segment (start 67.8815 30.1625) (end 68.326 30.607) (width 0.3) (layer "F.Cu") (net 6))
 (segment (start 66.04 25.527) (end 64.389 25.527) (width 0.3) (layer "F.Cu") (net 6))
 (segment (start 60.59 34.798) (end 60.452 34.66) (width 0.3) (layer "F.Cu") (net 6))
 (segment (start 69.207444 32.504444) (end 69.207444 34.028444) (width 0.3) (layer "F.Cu") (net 6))
 (segment (start 63.754 31.623) (end 63.754 30.607) (width 0.3) (layer "F.Cu") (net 6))
 (segment (start 62.087888 34.798) (end 60.59 34.798) (width 0.3) (layer "F.Cu") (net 6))
 (segment (start 64.643 30.607) (end 67.437 30.607) (width 0.3) (layer "F.Cu") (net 6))
 (segment (start 69.984556 34.805556) (end 71.482444 34.805556) (width 0.3) (layer "F.Cu") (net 6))
 (segment (start 68.326 31.623) (end 69.207444 32.504444) (width 0.3) (layer "F.Cu") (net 6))
 (via (at 69.207444 34.028444) (size 0.4) (drill 0.2) (layers "F.Cu" "B.Cu") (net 6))
 (via (at 62.603444 35.313556) (size 0.4) (drill 0.2) (layers "F.Cu" "B.Cu") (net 6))
 (via (at 66.04 25.527) (size 0.4) (drill 0.2) (layers "F.Cu" "B.Cu") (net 6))
 (via (at 69.984556 34.805556) (size 0.4) (drill 0.2) (layers "F.Cu" "B.Cu") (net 6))
 (via (at 64.516 27.051) (size 0.4) (drill 0.2) (layers "F.Cu" "B.Cu") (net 6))
 (via (at 63.380556 34.536444) (size 0.4) (drill 0.2) (layers "F.Cu" "B.Cu") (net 6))
 (segment (start 65.151 27.051) (end 66.04 26.162) (width 0.3) (layer "B.Cu") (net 6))
 (segment (start 62.603444 35.313556) (end 63.380556 34.536444) (width 0.3) (layer "B.Cu") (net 6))
 (segment (start 64.516 27.051) (end 65.151 27.051) (width 0.3) (layer "B.Cu") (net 6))
 (segment (start 66.04 26.162) (end 66.04 25.527) (width 0.3) (layer "B.Cu") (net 6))
 (segment (start 69.984556 34.805556) (end 69.207444 34.028444) (width 0.3) (layer "B.Cu") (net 6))
 (segment (start 64.008 41.402) (end 63.754 41.148) (width 0.3) (layer "F.Cu") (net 8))
 (segment (start 60.452 36.46) (end 60.452 38.354) (width 0.3) (layer "F.Cu") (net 8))
 (segment (start 66.04 41.402) (end 64.008 41.402) (width 0.3) (layer "F.Cu") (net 8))
 (segment (start 71.628 36.46) (end 71.628 38.354) (width 0.3) (layer "F.Cu") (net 8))
 (via (at 66.04 41.402) (size 0.4) (drill 0.2) (layers "F.Cu" "B.Cu") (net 8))
 (via (at 60.452 38.354) (size 0.4) (drill 0.2) (layers "F.Cu" "B.Cu") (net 8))
 (via (at 71.628 38.354) (size 0.4) (drill 0.2) (layers "F.Cu" "B.Cu") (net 8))
 (segment (start 60.452 38.354) (end 60.452 40.155492) (width 0.3) (layer "B.Cu") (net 8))
 (segment (start 70.358 41.402) (end 66.04 41.402) (width 0.3) (layer "B.Cu") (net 8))
 (segment (start 61.698508 41.402) (end 66.04 41.402) (width 0.3) (layer "B.Cu") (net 8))
 (segment (start 71.628 38.354) (end 71.628 40.132) (width 0.3) (layer "B.Cu") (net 8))
 (segment (start 60.452 40.155492) (end 61.698508 41.402) (width 0.3) (layer "B.Cu") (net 8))
 (segment (start 71.628 40.132) (end 70.358 41.402) (width 0.3) (layer "B.Cu") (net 8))
 (segment (start 71.617766 31.75) (end 70.612 31.75) (width 0.3) (layer "F.Cu") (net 5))
 (segment (start 69.85 34.163) (end 68.072 35.941) (width 0.3) (layer "F.Cu") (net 5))
 (segment (start 69.85 32.512) (end 69.85 34.163) (width 0.3) (layer "F.Cu") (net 5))
 (segment (start 70.612 31.75) (end 69.85 32.512) (width 0.3) (layer "F.Cu") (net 5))
 (segment (start 72.528 35.56) (end 72.39 35.698) (width 0.3) (layer "F.Cu") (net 5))
 (segment (start 68.072 35.941) (end 62.45307 35.941) (width 0.3) (layer "F.Cu") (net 5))
 (segment (start 72.39 35.422) (end 72.39 32.522234) (width 0.3) (layer "F.Cu") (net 5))
 (segment (start 72.528 35.56) (end 72.39 35.422) (width 0.3) (layer "F.Cu") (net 5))
 (segment (start 72.39 35.698) (end 72.39 39.116) (width 0.3) (layer "F.Cu") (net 5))
 (segment (start 62.45307 35.941) (end 62.07207 35.56) (width 0.3) (layer "F.Cu") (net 5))
 (segment (start 72.39 32.522234) (end 71.617766 31.75) (width 0.3) (layer "F.Cu") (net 5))
 (segment (start 62.07207 35.56) (end 61.352 35.56) (width 0.3) (layer "F.Cu") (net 5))
 (segment (start 72.39 39.116) (end 72.136 39.37) (width 0.3) (layer "F.Cu") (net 5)))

